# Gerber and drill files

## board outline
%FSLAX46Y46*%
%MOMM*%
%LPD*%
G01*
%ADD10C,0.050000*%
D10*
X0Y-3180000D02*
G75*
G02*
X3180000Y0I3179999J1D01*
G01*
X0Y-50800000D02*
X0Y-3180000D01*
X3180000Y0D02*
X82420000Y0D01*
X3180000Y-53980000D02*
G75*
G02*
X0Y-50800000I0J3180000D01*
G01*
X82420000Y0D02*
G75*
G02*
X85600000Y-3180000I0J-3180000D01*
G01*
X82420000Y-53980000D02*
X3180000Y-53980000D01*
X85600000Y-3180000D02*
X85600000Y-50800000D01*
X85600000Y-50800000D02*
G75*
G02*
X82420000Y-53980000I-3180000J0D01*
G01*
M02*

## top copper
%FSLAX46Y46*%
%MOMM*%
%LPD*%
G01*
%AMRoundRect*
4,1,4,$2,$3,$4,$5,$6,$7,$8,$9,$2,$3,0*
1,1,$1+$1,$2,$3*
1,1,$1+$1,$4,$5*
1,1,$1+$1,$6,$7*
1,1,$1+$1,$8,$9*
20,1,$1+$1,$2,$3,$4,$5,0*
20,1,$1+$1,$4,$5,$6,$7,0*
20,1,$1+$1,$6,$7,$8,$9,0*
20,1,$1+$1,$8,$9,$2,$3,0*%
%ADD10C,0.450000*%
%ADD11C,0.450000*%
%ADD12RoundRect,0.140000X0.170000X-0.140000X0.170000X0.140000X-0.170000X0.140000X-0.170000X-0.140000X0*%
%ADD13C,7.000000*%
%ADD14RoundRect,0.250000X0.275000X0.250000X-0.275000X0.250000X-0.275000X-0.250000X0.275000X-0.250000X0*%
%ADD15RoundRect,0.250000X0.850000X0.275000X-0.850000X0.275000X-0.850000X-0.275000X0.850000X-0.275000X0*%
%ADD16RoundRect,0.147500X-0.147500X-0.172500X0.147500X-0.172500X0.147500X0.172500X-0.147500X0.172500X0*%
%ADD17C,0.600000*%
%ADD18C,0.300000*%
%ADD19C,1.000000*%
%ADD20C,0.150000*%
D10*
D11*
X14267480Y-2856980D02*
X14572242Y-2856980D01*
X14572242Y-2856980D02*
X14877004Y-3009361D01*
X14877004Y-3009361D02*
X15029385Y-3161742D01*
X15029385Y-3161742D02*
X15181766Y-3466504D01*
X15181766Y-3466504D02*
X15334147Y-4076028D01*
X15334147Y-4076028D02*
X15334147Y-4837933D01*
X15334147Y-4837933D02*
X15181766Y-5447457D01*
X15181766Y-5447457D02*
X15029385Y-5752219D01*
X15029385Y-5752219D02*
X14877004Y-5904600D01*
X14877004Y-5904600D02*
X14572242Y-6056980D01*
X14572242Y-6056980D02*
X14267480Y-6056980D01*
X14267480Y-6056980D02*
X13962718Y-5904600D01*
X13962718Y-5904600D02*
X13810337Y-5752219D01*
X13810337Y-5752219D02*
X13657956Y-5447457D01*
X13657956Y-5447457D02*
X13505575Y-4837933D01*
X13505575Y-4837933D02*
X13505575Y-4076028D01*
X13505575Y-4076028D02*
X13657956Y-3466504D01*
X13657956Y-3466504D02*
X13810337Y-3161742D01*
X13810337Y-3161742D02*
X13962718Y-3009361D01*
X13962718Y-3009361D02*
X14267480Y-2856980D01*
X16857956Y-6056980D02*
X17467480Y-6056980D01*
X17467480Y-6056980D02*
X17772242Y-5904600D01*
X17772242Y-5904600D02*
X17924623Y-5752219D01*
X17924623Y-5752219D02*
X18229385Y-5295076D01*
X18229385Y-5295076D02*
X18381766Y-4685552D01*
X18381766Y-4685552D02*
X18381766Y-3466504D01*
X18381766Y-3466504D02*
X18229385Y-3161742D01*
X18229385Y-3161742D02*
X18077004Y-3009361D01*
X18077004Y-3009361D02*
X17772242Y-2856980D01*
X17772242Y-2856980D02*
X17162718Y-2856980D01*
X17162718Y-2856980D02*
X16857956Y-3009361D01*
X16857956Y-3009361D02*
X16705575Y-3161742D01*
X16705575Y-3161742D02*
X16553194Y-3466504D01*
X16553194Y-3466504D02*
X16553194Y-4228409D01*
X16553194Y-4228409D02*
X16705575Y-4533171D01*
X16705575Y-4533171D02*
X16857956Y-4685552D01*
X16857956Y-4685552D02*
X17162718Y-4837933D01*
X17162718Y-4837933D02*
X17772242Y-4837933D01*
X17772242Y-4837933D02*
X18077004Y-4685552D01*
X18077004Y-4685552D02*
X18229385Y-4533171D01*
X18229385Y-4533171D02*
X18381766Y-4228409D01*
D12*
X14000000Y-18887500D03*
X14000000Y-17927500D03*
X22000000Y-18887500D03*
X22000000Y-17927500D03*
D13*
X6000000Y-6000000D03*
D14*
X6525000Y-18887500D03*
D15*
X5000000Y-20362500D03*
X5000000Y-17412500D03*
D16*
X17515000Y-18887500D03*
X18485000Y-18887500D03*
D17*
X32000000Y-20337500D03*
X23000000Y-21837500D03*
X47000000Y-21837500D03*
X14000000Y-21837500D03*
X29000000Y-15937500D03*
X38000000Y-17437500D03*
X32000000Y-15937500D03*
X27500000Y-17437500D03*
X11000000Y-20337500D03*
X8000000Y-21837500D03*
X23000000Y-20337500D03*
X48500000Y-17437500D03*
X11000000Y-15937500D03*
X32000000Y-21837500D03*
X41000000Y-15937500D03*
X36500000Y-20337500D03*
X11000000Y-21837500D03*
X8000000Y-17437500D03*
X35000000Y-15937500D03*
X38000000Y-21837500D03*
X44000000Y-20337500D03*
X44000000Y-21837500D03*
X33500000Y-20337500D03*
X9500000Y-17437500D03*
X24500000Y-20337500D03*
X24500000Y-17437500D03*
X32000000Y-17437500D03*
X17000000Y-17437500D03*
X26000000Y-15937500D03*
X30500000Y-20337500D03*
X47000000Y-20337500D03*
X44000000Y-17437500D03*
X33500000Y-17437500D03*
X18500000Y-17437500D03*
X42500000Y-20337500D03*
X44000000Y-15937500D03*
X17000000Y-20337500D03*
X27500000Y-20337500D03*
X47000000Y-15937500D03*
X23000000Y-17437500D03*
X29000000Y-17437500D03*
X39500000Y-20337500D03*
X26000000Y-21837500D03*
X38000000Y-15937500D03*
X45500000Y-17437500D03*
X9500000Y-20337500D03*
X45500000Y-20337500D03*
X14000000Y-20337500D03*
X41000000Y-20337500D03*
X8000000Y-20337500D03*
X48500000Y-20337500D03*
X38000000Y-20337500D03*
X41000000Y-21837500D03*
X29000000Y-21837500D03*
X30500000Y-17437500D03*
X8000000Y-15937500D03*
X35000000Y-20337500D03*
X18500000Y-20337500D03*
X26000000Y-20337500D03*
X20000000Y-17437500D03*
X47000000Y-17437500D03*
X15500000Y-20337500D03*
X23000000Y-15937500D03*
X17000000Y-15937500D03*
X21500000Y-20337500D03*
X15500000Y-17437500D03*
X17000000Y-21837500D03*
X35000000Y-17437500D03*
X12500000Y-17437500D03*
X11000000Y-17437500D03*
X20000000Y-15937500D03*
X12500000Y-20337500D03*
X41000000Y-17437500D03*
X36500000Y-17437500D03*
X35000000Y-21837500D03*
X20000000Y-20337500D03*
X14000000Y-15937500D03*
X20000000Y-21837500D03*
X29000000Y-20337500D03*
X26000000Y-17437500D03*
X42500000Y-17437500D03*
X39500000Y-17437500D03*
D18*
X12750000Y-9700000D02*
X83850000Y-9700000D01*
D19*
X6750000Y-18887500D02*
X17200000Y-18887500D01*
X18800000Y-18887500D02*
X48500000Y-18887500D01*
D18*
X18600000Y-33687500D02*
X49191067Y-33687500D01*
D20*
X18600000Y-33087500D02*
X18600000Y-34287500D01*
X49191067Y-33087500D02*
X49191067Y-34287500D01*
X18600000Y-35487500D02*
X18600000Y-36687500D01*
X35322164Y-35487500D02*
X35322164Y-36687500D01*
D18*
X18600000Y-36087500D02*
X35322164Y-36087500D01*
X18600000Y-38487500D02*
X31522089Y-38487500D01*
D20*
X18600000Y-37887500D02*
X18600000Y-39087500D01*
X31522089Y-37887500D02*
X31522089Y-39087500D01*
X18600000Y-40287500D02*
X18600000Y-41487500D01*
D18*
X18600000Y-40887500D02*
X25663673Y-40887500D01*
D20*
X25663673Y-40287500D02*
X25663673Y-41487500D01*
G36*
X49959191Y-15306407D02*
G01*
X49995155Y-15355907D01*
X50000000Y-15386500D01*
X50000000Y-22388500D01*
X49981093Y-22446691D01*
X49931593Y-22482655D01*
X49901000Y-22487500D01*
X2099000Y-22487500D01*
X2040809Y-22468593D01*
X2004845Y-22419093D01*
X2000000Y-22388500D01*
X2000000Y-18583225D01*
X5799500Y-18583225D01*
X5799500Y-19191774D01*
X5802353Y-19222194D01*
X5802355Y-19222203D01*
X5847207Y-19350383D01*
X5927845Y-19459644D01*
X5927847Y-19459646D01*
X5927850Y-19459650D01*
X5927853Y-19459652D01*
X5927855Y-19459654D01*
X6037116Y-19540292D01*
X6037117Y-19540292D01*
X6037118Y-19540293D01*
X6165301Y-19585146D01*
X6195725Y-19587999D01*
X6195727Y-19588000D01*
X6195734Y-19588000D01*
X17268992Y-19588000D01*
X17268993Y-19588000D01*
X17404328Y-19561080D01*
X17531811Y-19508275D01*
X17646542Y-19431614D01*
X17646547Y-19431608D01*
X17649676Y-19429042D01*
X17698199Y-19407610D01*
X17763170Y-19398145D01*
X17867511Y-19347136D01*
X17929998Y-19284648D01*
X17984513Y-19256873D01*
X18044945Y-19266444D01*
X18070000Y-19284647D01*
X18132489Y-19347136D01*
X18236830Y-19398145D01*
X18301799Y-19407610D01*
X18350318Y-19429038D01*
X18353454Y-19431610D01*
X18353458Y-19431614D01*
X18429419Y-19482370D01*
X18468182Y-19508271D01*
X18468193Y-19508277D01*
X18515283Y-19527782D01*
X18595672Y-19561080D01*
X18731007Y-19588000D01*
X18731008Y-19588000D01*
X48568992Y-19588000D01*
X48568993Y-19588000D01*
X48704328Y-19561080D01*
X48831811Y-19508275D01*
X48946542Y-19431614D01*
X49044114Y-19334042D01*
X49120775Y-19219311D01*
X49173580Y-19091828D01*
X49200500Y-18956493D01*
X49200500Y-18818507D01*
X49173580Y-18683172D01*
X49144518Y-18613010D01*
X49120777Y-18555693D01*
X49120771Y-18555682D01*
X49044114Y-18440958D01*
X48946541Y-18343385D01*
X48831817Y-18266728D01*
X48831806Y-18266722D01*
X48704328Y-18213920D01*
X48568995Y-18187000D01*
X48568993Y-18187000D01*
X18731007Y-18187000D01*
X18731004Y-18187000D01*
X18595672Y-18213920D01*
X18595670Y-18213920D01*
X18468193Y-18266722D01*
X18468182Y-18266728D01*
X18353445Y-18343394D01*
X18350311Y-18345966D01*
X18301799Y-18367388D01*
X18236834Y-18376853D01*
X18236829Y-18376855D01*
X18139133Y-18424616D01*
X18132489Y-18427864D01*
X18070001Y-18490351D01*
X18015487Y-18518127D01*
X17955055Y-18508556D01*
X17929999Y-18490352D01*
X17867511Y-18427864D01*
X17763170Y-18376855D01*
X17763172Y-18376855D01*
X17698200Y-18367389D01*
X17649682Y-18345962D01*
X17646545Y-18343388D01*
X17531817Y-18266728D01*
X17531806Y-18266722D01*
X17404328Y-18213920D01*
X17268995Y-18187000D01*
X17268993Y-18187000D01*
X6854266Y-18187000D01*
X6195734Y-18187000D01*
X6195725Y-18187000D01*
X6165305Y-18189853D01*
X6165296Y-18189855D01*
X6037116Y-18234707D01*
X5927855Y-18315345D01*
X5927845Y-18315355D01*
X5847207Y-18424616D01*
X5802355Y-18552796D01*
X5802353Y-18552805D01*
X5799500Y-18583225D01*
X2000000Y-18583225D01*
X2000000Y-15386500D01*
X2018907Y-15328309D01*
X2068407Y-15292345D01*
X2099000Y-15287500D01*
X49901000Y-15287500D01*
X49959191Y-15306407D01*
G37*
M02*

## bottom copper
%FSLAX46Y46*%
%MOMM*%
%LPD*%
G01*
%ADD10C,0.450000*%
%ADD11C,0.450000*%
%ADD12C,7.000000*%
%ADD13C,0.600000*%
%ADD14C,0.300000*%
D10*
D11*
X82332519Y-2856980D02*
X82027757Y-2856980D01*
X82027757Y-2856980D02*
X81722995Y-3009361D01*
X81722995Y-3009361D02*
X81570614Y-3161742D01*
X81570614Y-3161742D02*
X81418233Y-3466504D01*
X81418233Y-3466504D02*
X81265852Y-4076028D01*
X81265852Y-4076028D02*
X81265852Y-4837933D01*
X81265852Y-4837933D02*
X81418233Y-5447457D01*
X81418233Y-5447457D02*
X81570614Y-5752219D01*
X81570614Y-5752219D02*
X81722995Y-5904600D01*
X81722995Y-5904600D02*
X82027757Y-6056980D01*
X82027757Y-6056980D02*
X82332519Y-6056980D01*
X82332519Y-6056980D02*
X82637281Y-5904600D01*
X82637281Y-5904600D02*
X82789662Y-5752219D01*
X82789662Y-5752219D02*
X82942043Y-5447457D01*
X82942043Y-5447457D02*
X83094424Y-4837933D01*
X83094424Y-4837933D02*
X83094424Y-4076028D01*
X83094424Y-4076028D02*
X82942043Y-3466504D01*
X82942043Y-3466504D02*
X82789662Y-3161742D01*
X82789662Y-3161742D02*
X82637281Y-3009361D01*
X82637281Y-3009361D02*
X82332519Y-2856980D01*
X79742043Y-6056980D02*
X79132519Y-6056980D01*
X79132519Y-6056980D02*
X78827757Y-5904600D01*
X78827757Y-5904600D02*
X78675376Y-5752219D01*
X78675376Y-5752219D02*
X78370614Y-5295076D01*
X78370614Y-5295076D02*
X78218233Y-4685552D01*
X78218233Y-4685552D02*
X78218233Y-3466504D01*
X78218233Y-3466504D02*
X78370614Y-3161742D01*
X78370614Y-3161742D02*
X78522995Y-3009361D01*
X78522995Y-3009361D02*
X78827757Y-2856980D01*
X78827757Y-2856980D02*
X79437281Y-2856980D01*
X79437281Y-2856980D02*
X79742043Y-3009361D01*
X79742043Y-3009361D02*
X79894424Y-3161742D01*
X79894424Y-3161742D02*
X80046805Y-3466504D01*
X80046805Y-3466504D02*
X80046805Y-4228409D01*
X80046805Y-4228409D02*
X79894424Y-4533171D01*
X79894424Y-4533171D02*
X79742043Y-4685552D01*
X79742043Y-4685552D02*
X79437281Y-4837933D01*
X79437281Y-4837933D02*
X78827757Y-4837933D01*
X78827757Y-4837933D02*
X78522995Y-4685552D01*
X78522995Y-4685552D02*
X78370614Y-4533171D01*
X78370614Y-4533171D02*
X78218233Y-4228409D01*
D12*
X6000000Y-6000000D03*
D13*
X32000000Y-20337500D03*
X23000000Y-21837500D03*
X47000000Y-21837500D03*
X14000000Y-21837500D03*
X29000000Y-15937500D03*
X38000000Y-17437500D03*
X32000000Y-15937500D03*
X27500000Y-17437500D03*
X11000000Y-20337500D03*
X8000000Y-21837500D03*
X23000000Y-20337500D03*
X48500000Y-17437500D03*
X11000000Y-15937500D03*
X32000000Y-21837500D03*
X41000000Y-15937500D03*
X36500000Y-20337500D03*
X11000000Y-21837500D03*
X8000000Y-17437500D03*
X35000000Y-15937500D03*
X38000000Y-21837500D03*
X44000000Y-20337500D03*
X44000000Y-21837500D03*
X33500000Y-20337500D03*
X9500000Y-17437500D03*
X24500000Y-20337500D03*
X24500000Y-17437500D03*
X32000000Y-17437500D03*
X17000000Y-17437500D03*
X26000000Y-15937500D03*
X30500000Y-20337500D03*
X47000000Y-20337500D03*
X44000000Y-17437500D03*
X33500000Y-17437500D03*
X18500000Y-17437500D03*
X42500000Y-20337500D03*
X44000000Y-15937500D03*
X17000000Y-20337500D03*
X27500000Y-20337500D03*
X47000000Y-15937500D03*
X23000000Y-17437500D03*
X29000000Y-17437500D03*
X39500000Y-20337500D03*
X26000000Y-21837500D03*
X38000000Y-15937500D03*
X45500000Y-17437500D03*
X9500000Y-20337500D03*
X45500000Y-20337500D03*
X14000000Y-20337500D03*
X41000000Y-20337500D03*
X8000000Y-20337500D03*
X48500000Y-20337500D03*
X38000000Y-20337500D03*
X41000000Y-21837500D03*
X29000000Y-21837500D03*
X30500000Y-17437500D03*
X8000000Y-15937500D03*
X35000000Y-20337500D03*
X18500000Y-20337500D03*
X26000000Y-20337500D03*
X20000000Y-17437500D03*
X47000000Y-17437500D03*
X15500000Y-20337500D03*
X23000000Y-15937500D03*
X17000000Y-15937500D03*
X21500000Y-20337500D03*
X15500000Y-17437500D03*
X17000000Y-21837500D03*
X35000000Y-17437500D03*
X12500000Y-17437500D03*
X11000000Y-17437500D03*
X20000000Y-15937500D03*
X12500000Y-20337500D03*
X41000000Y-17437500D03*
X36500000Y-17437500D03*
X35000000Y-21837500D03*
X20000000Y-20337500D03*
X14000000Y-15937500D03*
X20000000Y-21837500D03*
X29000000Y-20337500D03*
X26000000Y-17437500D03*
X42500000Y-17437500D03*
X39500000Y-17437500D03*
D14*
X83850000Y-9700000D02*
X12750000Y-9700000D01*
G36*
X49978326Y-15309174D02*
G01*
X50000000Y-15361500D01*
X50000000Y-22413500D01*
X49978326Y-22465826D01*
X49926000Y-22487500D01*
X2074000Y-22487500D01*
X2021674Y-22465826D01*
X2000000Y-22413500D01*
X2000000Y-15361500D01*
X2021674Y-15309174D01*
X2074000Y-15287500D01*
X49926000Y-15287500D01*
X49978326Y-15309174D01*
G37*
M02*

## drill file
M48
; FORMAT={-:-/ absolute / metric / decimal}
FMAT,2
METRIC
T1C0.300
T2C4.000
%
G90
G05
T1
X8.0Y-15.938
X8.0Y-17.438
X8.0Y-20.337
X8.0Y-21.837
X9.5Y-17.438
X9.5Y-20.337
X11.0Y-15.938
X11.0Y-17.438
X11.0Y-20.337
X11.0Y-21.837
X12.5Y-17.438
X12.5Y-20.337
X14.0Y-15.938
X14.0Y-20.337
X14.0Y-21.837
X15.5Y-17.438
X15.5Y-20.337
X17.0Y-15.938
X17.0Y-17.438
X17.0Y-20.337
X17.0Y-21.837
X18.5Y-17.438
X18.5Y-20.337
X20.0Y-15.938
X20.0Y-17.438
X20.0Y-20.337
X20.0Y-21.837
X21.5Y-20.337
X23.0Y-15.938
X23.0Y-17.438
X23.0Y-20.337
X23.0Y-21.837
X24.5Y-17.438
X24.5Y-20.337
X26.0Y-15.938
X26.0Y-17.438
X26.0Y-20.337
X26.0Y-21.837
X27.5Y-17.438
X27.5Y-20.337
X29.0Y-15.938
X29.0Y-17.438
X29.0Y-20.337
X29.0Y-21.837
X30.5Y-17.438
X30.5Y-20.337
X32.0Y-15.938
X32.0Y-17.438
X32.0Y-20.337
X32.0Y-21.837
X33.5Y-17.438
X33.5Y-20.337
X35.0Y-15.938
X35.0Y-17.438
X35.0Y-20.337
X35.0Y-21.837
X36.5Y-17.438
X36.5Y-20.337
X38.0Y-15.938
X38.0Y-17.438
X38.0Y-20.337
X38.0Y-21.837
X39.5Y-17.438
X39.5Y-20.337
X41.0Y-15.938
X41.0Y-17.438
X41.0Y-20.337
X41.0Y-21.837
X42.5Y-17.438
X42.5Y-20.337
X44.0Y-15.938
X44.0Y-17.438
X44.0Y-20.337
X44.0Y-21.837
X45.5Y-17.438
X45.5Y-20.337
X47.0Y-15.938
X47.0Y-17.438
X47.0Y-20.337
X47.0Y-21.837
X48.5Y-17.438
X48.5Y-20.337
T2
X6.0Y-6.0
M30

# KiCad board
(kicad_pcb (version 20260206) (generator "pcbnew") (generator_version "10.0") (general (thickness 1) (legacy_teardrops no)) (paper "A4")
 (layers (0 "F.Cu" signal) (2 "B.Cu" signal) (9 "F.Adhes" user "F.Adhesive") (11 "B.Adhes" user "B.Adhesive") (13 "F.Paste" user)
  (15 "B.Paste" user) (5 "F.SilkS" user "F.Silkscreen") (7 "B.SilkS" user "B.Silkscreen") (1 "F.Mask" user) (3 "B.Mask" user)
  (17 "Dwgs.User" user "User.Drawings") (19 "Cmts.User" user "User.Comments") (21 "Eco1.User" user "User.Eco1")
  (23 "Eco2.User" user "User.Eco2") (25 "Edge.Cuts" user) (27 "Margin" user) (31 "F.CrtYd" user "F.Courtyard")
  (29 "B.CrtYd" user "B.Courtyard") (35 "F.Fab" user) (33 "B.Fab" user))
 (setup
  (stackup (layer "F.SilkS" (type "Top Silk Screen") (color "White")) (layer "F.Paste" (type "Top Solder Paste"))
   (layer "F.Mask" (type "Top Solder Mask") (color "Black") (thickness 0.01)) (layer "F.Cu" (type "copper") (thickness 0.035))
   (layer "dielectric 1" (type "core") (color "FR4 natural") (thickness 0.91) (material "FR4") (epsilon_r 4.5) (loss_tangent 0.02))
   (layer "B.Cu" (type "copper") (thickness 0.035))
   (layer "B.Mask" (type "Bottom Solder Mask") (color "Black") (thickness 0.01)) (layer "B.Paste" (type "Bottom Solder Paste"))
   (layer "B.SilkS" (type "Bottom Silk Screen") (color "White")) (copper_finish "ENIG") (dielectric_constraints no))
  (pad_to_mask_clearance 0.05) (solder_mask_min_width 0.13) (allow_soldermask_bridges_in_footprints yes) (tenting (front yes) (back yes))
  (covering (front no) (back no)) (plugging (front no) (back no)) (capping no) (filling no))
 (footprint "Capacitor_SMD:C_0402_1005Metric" (layer "F.Cu") (at 14 18.4075 90)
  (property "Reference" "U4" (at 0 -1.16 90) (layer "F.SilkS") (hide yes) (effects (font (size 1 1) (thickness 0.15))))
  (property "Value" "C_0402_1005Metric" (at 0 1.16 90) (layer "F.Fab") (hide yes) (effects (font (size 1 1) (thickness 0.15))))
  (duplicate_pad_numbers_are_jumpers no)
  (pad "1" smd roundrect (at -0.48 0 90) (size 0.56 0.62) (layers "F.Cu" "F.Mask") (roundrect_rratio 0.25) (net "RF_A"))
  (pad "2" smd roundrect (at 0.48 0 90) (size 0.56 0.62) (layers "F.Cu" "F.Mask") (roundrect_rratio 0.25) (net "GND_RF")))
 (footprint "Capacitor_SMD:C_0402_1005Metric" (layer "F.Cu") (at 22 18.4075 90)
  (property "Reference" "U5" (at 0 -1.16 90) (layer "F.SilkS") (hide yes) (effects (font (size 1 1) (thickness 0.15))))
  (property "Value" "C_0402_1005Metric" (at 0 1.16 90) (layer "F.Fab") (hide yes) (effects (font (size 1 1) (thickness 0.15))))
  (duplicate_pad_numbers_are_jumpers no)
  (pad "1" smd roundrect (at -0.48 0 90) (size 0.56 0.62) (layers "F.Cu" "F.Mask") (roundrect_rratio 0.25) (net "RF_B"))
  (pad "2" smd roundrect (at 0.48 0 90) (size 0.56 0.62) (layers "F.Cu" "F.Mask") (roundrect_rratio 0.25) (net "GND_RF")))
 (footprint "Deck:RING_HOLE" (layer "F.Cu") (at 6 6)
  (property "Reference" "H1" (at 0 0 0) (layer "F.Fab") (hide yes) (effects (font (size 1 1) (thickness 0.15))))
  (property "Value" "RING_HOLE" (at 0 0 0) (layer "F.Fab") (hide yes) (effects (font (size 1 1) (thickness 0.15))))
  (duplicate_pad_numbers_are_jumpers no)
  (pad "" thru_hole circle (at 0 0) (size 7 7) (drill 4) (layers "*.Cu" "*.Mask") (remove_unused_layers no)))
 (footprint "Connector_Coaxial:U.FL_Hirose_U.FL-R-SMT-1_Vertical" (layer "F.Cu") (at 5 18.8875 180)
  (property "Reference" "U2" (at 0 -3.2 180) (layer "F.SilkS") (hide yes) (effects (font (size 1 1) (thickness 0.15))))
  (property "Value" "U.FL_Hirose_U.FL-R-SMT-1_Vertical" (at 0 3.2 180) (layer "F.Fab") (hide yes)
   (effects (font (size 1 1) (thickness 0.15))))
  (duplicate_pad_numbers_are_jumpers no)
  (pad "1" smd roundrect (at -1.525 0 180) (size 1.05 1) (layers "F.Cu" "F.Mask") (roundrect_rratio 0.25) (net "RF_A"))
  (pad "2" smd roundrect (at 0 -1.475 180) (size 2.2 1.05) (layers "F.Cu" "F.Mask") (roundrect_rratio 0.2380952381) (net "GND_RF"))
  (pad "2" smd roundrect (at 0 1.475 180) (size 2.2 1.05) (layers "F.Cu" "F.Mask") (roundrect_rratio 0.2380952381) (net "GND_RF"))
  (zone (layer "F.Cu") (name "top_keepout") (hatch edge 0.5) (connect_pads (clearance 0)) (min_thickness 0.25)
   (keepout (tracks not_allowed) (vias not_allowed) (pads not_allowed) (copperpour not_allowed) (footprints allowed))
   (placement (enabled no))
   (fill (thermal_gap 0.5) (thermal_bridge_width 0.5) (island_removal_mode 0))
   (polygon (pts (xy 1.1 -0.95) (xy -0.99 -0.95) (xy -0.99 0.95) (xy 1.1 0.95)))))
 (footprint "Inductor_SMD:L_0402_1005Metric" (layer "F.Cu") (at 18 18.8875)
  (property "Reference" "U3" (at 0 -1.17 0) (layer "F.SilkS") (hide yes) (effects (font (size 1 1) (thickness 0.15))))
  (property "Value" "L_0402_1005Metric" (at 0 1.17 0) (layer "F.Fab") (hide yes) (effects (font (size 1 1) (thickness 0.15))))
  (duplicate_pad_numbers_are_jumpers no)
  (pad "1" smd roundrect (at -0.485 0) (size 0.59 0.64) (layers "F.Cu" "F.Mask") (roundrect_rratio 0.25) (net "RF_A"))
  (pad "2" smd roundrect (at 0.485 0) (size 0.59 0.64) (layers "F.Cu" "F.Mask") (roundrect_rratio 0.25) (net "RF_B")))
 (gr_arc (start 0 3.18) (mid 0.9314 0.9314) (end 3.18 0) (stroke (width 0.05) (type solid)) (layer "Edge.Cuts"))
 (gr_line (start 0 50.8) (end 0 3.18) (stroke (width 0.05) (type solid)) (layer "Edge.Cuts"))
 (gr_line (start 3.18 0) (end 82.42 0) (stroke (width 0.05) (type solid)) (layer "Edge.Cuts"))
 (gr_arc (start 3.18 53.98) (mid 0.9314 53.0486) (end 0 50.8) (stroke (width 0.05) (type solid)) (layer "Edge.Cuts"))
 (gr_arc (start 82.42 0) (mid 84.6686 0.9314) (end 85.6 3.18) (stroke (width 0.05) (type solid)) (layer "Edge.Cuts"))
 (gr_line (start 82.42 53.98) (end 3.18 53.98) (stroke (width 0.05) (type solid)) (layer "Edge.Cuts"))
 (gr_line (start 85.6 3.18) (end 85.6 50.8) (stroke (width 0.05) (type solid)) (layer "Edge.Cuts"))
 (gr_arc (start 85.6 50.8) (mid 84.6686 53.0486) (end 82.42 53.98) (stroke (width 0.05) (type solid)) (layer "Edge.Cuts"))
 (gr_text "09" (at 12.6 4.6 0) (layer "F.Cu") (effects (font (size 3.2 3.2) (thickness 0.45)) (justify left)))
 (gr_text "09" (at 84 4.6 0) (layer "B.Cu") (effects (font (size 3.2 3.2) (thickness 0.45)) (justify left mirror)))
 (segment (start 12.75 9.7) (end 83.85 9.7) (width 0.3) (layer "F.Cu") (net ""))
 (segment (start 83.85 9.7) (end 12.75 9.7) (width 0.3) (layer "B.Cu") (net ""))
 (segment (start 6.75 18.8875) (end 17.2 18.8875) (width 1) (layer "F.Cu") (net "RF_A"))
 (via (at 32 20.3375) (size 0.6) (drill 0.3) (layers "F.Cu" "B.Cu") (tenting (front no) (back no)) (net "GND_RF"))
 (via (at 23 21.8375) (size 0.6) (drill 0.3) (layers "F.Cu" "B.Cu") (tenting (front no) (back no)) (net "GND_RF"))
 (via (at 47 21.8375) (size 0.6) (drill 0.3) (layers "F.Cu" "B.Cu") (tenting (front no) (back no)) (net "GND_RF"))
 (via (at 14 21.8375) (size 0.6) (drill 0.3) (layers "F.Cu" "B.Cu") (tenting (front no) (back no)) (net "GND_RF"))
 (via (at 29 15.9375) (size 0.6) (drill 0.3) (layers "F.Cu" "B.Cu") (tenting (front no) (back no)) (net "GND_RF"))
 (via (at 38 17.4375) (size 0.6) (drill 0.3) (layers "F.Cu" "B.Cu") (tenting (front no) (back no)) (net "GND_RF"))
 (via (at 32 15.9375) (size 0.6) (drill 0.3) (layers "F.Cu" "B.Cu") (tenting (front no) (back no)) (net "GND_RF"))
 (via (at 27.5 17.4375) (size 0.6) (drill 0.3) (layers "F.Cu" "B.Cu") (tenting (front no) (back no)) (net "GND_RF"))
 (via (at 11 20.3375) (size 0.6) (drill 0.3) (layers "F.Cu" "B.Cu") (tenting (front no) (back no)) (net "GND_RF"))
 (via (at 8 21.8375) (size 0.6) (drill 0.3) (layers "F.Cu" "B.Cu") (tenting (front no) (back no)) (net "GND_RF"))
 (via (at 23 20.3375) (size 0.6) (drill 0.3) (layers "F.Cu" "B.Cu") (tenting (front no) (back no)) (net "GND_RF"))
 (via (at 48.5 17.4375) (size 0.6) (drill 0.3) (layers "F.Cu" "B.Cu") (tenting (front no) (back no)) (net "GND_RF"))
 (via (at 11 15.9375) (size 0.6) (drill 0.3) (layers "F.Cu" "B.Cu") (tenting (front no) (back no)) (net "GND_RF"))
 (via (at 32 21.8375) (size 0.6) (drill 0.3) (layers "F.Cu" "B.Cu") (tenting (front no) (back no)) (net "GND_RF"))
 (via (at 41 15.9375) (size 0.6) (drill 0.3) (layers "F.Cu" "B.Cu") (tenting (front no) (back no)) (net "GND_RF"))
 (via (at 36.5 20.3375) (size 0.6) (drill 0.3) (layers "F.Cu" "B.Cu") (tenting (front no) (back no)) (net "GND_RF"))
 (via (at 11 21.8375) (size 0.6) (drill 0.3) (layers "F.Cu" "B.Cu") (tenting (front no) (back no)) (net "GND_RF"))
 (via (at 8 17.4375) (size 0.6) (drill 0.3) (layers "F.Cu" "B.Cu") (tenting (front no) (back no)) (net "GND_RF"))
 (via (at 35 15.9375) (size 0.6) (drill 0.3) (layers "F.Cu" "B.Cu") (tenting (front no) (back no)) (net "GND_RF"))
 (via (at 38 21.8375) (size 0.6) (drill 0.3) (layers "F.Cu" "B.Cu") (tenting (front no) (back no)) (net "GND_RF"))
 (via (at 44 20.3375) (size 0.6) (drill 0.3) (layers "F.Cu" "B.Cu") (tenting (front no) (back no)) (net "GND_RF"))
 (via (at 44 21.8375) (size 0.6) (drill 0.3) (layers "F.Cu" "B.Cu") (tenting (front no) (back no)) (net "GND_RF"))
 (via (at 33.5 20.3375) (size 0.6) (drill 0.3) (layers "F.Cu" "B.Cu") (tenting (front no) (back no)) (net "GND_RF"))
 (via (at 9.5 17.4375) (size 0.6) (drill 0.3) (layers "F.Cu" "B.Cu") (tenting (front no) (back no)) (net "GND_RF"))
 (via (at 24.5 20.3375) (size 0.6) (drill 0.3) (layers "F.Cu" "B.Cu") (tenting (front no) (back no)) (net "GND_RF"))
 (via (at 24.5 17.4375) (size 0.6) (drill 0.3) (layers "F.Cu" "B.Cu") (tenting (front no) (back no)) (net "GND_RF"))
 (via (at 32 17.4375) (size 0.6) (drill 0.3) (layers "F.Cu" "B.Cu") (tenting (front no) (back no)) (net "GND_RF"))
 (via (at 17 17.4375) (size 0.6) (drill 0.3) (layers "F.Cu" "B.Cu") (tenting (front no) (back no)) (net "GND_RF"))
 (via (at 26 15.9375) (size 0.6) (drill 0.3) (layers "F.Cu" "B.Cu") (tenting (front no) (back no)) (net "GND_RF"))
 (via (at 30.5 20.3375) (size 0.6) (drill 0.3) (layers "F.Cu" "B.Cu") (tenting (front no) (back no)) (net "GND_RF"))
 (via (at 47 20.3375) (size 0.6) (drill 0.3) (layers "F.Cu" "B.Cu") (tenting (front no) (back no)) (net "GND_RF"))
 (via (at 44 17.4375) (size 0.6) (drill 0.3) (layers "F.Cu" "B.Cu") (tenting (front no) (back no)) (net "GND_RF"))
 (via (at 33.5 17.4375) (size 0.6) (drill 0.3) (layers "F.Cu" "B.Cu") (tenting (front no) (back no)) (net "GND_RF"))
 (via (at 18.5 17.4375) (size 0.6) (drill 0.3) (layers "F.Cu" "B.Cu") (tenting (front no) (back no)) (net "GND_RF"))
 (via (at 42.5 20.3375) (size 0.6) (drill 0.3) (layers "F.Cu" "B.Cu") (tenting (front no) (back no)) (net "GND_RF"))
 (via (at 44 15.9375) (size 0.6) (drill 0.3) (layers "F.Cu" "B.Cu") (tenting (front no) (back no)) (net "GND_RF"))
 (via (at 17 20.3375) (size 0.6) (drill 0.3) (layers "F.Cu" "B.Cu") (tenting (front no) (back no)) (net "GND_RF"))
 (via (at 27.5 20.3375) (size 0.6) (drill 0.3) (layers "F.Cu" "B.Cu") (tenting (front no) (back no)) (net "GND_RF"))
 (via (at 47 15.9375) (size 0.6) (drill 0.3) (layers "F.Cu" "B.Cu") (tenting (front no) (back no)) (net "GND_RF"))
 (via (at 23 17.4375) (size 0.6) (drill 0.3) (layers "F.Cu" "B.Cu") (tenting (front no) (back no)) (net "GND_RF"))
 (via (at 29 17.4375) (size 0.6) (drill 0.3) (layers "F.Cu" "B.Cu") (tenting (front no) (back no)) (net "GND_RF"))
 (via (at 39.5 20.3375) (size 0.6) (drill 0.3) (layers "F.Cu" "B.Cu") (tenting (front no) (back no)) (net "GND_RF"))
 (via (at 26 21.8375) (size 0.6) (drill 0.3) (layers "F.Cu" "B.Cu") (tenting (front no) (back no)) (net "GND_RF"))
 (via (at 38 15.9375) (size 0.6) (drill 0.3) (layers "F.Cu" "B.Cu") (tenting (front no) (back no)) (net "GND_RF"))
 (via (at 45.5 17.4375) (size 0.6) (drill 0.3) (layers "F.Cu" "B.Cu") (tenting (front no) (back no)) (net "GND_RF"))
 (via (at 9.5 20.3375) (size 0.6) (drill 0.3) (layers "F.Cu" "B.Cu") (tenting (front no) (back no)) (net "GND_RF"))
 (via (at 45.5 20.3375) (size 0.6) (drill 0.3) (layers "F.Cu" "B.Cu") (tenting (front no) (back no)) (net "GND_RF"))
 (via (at 14 20.3375) (size 0.6) (drill 0.3) (layers "F.Cu" "B.Cu") (tenting (front no) (back no)) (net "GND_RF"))
 (via (at 41 20.3375) (size 0.6) (drill 0.3) (layers "F.Cu" "B.Cu") (tenting (front no) (back no)) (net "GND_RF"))
 (via (at 8 20.3375) (size 0.6) (drill 0.3) (layers "F.Cu" "B.Cu") (tenting (front no) (back no)) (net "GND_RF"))
 (via (at 48.5 20.3375) (size 0.6) (drill 0.3) (layers "F.Cu" "B.Cu") (tenting (front no) (back no)) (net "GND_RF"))
 (via (at 38 20.3375) (size 0.6) (drill 0.3) (layers "F.Cu" "B.Cu") (tenting (front no) (back no)) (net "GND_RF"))
 (via (at 41 21.8375) (size 0.6) (drill 0.3) (layers "F.Cu" "B.Cu") (tenting (front no) (back no)) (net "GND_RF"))
 (via (at 29 21.8375) (size 0.6) (drill 0.3) (layers "F.Cu" "B.Cu") (tenting (front no) (back no)) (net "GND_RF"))
 (via (at 30.5 17.4375) (size 0.6) (drill 0.3) (layers "F.Cu" "B.Cu") (tenting (front no) (back no)) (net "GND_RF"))
 (via (at 8 15.9375) (size 0.6) (drill 0.3) (layers "F.Cu" "B.Cu") (tenting (front no) (back no)) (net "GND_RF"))
 (via (at 35 20.3375) (size 0.6) (drill 0.3) (layers "F.Cu" "B.Cu") (tenting (front no) (back no)) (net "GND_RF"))
 (via (at 18.5 20.3375) (size 0.6) (drill 0.3) (layers "F.Cu" "B.Cu") (tenting (front no) (back no)) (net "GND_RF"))
 (via (at 26 20.3375) (size 0.6) (drill 0.3) (layers "F.Cu" "B.Cu") (tenting (front no) (back no)) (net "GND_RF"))
 (via (at 20 17.4375) (size 0.6) (drill 0.3) (layers "F.Cu" "B.Cu") (tenting (front no) (back no)) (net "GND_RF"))
 (via (at 47 17.4375) (size 0.6) (drill 0.3) (layers "F.Cu" "B.Cu") (tenting (front no) (back no)) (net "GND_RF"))
 (via (at 15.5 20.3375) (size 0.6) (drill 0.3) (layers "F.Cu" "B.Cu") (tenting (front no) (back no)) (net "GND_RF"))
 (via (at 23 15.9375) (size 0.6) (drill 0.3) (layers "F.Cu" "B.Cu") (tenting (front no) (back no)) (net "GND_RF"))
 (via (at 17 15.9375) (size 0.6) (drill 0.3) (layers "F.Cu" "B.Cu") (tenting (front no) (back no)) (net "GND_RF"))
 (via (at 21.5 20.3375) (size 0.6) (drill 0.3) (layers "F.Cu" "B.Cu") (tenting (front no) (back no)) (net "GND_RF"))
 (via (at 15.5 17.4375) (size 0.6) (drill 0.3) (layers "F.Cu" "B.Cu") (tenting (front no) (back no)) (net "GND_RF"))
 (via (at 17 21.8375) (size 0.6) (drill 0.3) (layers "F.Cu" "B.Cu") (tenting (front no) (back no)) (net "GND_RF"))
 (via (at 35 17.4375) (size 0.6) (drill 0.3) (layers "F.Cu" "B.Cu") (tenting (front no) (back no)) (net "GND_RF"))
 (via (at 12.5 17.4375) (size 0.6) (drill 0.3) (layers "F.Cu" "B.Cu") (tenting (front no) (back no)) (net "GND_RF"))
 (via (at 11 17.4375) (size 0.6) (drill 0.3) (layers "F.Cu" "B.Cu") (tenting (front no) (back no)) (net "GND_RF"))
 (via (at 20 15.9375) (size 0.6) (drill 0.3) (layers "F.Cu" "B.Cu") (tenting (front no) (back no)) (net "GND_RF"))
 (via (at 12.5 20.3375) (size 0.6) (drill 0.3) (layers "F.Cu" "B.Cu") (tenting (front no) (back no)) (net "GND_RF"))
 (via (at 41 17.4375) (size 0.6) (drill 0.3) (layers "F.Cu" "B.Cu") (tenting (front no) (back no)) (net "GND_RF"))
 (via (at 36.5 17.4375) (size 0.6) (drill 0.3) (layers "F.Cu" "B.Cu") (tenting (front no) (back no)) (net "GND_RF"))
 (via (at 35 21.8375) (size 0.6) (drill 0.3) (layers "F.Cu" "B.Cu") (tenting (front no) (back no)) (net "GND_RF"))
 (via (at 20 20.3375) (size 0.6) (drill 0.3) (layers "F.Cu" "B.Cu") (tenting (front no) (back no)) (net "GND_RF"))
 (via (at 14 15.9375) (size 0.6) (drill 0.3) (layers "F.Cu" "B.Cu") (tenting (front no) (back no)) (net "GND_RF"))
 (via (at 20 21.8375) (size 0.6) (drill 0.3) (layers "F.Cu" "B.Cu") (tenting (front no) (back no)) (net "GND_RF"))
 (via (at 29 20.3375) (size 0.6) (drill 0.3) (layers "F.Cu" "B.Cu") (tenting (front no) (back no)) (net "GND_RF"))
 (via (at 26 17.4375) (size 0.6) (drill 0.3) (layers "F.Cu" "B.Cu") (tenting (front no) (back no)) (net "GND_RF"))
 (via (at 42.5 17.4375) (size 0.6) (drill 0.3) (layers "F.Cu" "B.Cu") (tenting (front no) (back no)) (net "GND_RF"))
 (via (at 39.5 17.4375) (size 0.6) (drill 0.3) (layers "F.Cu" "B.Cu") (tenting (front no) (back no)) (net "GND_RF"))
 (segment (start 18.8 18.8875) (end 48.5 18.8875) (width 1) (layer "F.Cu") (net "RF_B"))
 (segment (start 18.6 33.6875) (end 49.191067 33.6875) (width 0.3) (layer "F.Cu") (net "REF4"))
 (segment (start 18.6 33.0875) (end 18.6 34.2875) (width 0.15) (layer "F.Cu") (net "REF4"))
 (segment (start 49.191067 33.0875) (end 49.191067 34.2875) (width 0.15) (layer "F.Cu") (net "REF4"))
 (segment (start 18.6 35.4875) (end 18.6 36.6875) (width 0.15) (layer "F.Cu") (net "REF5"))
 (segment (start 35.322164 35.4875) (end 35.322164 36.6875) (width 0.15) (layer "F.Cu") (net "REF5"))
 (segment (start 18.6 36.0875) (end 35.322164 36.0875) (width 0.3) (layer "F.Cu") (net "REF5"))
 (segment (start 18.6 38.4875) (end 31.522089 38.4875) (width 0.3) (layer "F.Cu") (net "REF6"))
 (segment (start 18.6 37.8875) (end 18.6 39.0875) (width 0.15) (layer "F.Cu") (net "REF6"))
 (segment (start 31.522089 37.8875) (end 31.522089 39.0875) (width 0.15) (layer "F.Cu") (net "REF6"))
 (segment (start 18.6 40.2875) (end 18.6 41.4875) (width 0.15) (layer "F.Cu") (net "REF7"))
 (segment (start 18.6 40.8875) (end 25.663673 40.8875) (width 0.3) (layer "F.Cu") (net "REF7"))
 (segment (start 25.663673 40.2875) (end 25.663673 41.4875) (width 0.15) (layer "F.Cu") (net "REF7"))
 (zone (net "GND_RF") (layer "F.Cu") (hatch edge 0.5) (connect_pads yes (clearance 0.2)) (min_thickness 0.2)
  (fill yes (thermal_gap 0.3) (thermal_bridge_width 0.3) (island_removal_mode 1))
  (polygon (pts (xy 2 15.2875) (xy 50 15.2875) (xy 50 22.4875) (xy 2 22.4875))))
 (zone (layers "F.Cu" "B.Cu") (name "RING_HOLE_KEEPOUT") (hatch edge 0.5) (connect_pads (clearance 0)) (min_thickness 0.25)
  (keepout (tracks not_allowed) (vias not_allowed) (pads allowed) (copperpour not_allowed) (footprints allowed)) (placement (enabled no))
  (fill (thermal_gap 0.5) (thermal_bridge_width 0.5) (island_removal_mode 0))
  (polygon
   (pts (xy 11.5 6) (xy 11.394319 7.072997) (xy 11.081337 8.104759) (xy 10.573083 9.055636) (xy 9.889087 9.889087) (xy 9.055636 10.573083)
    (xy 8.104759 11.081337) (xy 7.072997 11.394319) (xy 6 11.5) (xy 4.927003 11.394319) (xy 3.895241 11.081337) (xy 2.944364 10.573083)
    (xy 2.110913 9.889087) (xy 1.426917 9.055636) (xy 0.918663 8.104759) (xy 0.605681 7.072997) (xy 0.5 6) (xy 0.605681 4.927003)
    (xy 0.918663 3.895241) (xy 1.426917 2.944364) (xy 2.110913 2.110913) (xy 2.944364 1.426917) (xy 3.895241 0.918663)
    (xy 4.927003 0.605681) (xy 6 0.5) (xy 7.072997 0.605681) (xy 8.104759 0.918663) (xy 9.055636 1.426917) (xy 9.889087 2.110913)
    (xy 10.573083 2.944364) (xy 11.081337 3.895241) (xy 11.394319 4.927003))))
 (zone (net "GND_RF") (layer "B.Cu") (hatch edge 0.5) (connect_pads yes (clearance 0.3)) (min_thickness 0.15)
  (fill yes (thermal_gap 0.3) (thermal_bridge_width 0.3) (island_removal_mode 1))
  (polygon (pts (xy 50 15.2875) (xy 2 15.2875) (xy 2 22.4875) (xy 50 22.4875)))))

